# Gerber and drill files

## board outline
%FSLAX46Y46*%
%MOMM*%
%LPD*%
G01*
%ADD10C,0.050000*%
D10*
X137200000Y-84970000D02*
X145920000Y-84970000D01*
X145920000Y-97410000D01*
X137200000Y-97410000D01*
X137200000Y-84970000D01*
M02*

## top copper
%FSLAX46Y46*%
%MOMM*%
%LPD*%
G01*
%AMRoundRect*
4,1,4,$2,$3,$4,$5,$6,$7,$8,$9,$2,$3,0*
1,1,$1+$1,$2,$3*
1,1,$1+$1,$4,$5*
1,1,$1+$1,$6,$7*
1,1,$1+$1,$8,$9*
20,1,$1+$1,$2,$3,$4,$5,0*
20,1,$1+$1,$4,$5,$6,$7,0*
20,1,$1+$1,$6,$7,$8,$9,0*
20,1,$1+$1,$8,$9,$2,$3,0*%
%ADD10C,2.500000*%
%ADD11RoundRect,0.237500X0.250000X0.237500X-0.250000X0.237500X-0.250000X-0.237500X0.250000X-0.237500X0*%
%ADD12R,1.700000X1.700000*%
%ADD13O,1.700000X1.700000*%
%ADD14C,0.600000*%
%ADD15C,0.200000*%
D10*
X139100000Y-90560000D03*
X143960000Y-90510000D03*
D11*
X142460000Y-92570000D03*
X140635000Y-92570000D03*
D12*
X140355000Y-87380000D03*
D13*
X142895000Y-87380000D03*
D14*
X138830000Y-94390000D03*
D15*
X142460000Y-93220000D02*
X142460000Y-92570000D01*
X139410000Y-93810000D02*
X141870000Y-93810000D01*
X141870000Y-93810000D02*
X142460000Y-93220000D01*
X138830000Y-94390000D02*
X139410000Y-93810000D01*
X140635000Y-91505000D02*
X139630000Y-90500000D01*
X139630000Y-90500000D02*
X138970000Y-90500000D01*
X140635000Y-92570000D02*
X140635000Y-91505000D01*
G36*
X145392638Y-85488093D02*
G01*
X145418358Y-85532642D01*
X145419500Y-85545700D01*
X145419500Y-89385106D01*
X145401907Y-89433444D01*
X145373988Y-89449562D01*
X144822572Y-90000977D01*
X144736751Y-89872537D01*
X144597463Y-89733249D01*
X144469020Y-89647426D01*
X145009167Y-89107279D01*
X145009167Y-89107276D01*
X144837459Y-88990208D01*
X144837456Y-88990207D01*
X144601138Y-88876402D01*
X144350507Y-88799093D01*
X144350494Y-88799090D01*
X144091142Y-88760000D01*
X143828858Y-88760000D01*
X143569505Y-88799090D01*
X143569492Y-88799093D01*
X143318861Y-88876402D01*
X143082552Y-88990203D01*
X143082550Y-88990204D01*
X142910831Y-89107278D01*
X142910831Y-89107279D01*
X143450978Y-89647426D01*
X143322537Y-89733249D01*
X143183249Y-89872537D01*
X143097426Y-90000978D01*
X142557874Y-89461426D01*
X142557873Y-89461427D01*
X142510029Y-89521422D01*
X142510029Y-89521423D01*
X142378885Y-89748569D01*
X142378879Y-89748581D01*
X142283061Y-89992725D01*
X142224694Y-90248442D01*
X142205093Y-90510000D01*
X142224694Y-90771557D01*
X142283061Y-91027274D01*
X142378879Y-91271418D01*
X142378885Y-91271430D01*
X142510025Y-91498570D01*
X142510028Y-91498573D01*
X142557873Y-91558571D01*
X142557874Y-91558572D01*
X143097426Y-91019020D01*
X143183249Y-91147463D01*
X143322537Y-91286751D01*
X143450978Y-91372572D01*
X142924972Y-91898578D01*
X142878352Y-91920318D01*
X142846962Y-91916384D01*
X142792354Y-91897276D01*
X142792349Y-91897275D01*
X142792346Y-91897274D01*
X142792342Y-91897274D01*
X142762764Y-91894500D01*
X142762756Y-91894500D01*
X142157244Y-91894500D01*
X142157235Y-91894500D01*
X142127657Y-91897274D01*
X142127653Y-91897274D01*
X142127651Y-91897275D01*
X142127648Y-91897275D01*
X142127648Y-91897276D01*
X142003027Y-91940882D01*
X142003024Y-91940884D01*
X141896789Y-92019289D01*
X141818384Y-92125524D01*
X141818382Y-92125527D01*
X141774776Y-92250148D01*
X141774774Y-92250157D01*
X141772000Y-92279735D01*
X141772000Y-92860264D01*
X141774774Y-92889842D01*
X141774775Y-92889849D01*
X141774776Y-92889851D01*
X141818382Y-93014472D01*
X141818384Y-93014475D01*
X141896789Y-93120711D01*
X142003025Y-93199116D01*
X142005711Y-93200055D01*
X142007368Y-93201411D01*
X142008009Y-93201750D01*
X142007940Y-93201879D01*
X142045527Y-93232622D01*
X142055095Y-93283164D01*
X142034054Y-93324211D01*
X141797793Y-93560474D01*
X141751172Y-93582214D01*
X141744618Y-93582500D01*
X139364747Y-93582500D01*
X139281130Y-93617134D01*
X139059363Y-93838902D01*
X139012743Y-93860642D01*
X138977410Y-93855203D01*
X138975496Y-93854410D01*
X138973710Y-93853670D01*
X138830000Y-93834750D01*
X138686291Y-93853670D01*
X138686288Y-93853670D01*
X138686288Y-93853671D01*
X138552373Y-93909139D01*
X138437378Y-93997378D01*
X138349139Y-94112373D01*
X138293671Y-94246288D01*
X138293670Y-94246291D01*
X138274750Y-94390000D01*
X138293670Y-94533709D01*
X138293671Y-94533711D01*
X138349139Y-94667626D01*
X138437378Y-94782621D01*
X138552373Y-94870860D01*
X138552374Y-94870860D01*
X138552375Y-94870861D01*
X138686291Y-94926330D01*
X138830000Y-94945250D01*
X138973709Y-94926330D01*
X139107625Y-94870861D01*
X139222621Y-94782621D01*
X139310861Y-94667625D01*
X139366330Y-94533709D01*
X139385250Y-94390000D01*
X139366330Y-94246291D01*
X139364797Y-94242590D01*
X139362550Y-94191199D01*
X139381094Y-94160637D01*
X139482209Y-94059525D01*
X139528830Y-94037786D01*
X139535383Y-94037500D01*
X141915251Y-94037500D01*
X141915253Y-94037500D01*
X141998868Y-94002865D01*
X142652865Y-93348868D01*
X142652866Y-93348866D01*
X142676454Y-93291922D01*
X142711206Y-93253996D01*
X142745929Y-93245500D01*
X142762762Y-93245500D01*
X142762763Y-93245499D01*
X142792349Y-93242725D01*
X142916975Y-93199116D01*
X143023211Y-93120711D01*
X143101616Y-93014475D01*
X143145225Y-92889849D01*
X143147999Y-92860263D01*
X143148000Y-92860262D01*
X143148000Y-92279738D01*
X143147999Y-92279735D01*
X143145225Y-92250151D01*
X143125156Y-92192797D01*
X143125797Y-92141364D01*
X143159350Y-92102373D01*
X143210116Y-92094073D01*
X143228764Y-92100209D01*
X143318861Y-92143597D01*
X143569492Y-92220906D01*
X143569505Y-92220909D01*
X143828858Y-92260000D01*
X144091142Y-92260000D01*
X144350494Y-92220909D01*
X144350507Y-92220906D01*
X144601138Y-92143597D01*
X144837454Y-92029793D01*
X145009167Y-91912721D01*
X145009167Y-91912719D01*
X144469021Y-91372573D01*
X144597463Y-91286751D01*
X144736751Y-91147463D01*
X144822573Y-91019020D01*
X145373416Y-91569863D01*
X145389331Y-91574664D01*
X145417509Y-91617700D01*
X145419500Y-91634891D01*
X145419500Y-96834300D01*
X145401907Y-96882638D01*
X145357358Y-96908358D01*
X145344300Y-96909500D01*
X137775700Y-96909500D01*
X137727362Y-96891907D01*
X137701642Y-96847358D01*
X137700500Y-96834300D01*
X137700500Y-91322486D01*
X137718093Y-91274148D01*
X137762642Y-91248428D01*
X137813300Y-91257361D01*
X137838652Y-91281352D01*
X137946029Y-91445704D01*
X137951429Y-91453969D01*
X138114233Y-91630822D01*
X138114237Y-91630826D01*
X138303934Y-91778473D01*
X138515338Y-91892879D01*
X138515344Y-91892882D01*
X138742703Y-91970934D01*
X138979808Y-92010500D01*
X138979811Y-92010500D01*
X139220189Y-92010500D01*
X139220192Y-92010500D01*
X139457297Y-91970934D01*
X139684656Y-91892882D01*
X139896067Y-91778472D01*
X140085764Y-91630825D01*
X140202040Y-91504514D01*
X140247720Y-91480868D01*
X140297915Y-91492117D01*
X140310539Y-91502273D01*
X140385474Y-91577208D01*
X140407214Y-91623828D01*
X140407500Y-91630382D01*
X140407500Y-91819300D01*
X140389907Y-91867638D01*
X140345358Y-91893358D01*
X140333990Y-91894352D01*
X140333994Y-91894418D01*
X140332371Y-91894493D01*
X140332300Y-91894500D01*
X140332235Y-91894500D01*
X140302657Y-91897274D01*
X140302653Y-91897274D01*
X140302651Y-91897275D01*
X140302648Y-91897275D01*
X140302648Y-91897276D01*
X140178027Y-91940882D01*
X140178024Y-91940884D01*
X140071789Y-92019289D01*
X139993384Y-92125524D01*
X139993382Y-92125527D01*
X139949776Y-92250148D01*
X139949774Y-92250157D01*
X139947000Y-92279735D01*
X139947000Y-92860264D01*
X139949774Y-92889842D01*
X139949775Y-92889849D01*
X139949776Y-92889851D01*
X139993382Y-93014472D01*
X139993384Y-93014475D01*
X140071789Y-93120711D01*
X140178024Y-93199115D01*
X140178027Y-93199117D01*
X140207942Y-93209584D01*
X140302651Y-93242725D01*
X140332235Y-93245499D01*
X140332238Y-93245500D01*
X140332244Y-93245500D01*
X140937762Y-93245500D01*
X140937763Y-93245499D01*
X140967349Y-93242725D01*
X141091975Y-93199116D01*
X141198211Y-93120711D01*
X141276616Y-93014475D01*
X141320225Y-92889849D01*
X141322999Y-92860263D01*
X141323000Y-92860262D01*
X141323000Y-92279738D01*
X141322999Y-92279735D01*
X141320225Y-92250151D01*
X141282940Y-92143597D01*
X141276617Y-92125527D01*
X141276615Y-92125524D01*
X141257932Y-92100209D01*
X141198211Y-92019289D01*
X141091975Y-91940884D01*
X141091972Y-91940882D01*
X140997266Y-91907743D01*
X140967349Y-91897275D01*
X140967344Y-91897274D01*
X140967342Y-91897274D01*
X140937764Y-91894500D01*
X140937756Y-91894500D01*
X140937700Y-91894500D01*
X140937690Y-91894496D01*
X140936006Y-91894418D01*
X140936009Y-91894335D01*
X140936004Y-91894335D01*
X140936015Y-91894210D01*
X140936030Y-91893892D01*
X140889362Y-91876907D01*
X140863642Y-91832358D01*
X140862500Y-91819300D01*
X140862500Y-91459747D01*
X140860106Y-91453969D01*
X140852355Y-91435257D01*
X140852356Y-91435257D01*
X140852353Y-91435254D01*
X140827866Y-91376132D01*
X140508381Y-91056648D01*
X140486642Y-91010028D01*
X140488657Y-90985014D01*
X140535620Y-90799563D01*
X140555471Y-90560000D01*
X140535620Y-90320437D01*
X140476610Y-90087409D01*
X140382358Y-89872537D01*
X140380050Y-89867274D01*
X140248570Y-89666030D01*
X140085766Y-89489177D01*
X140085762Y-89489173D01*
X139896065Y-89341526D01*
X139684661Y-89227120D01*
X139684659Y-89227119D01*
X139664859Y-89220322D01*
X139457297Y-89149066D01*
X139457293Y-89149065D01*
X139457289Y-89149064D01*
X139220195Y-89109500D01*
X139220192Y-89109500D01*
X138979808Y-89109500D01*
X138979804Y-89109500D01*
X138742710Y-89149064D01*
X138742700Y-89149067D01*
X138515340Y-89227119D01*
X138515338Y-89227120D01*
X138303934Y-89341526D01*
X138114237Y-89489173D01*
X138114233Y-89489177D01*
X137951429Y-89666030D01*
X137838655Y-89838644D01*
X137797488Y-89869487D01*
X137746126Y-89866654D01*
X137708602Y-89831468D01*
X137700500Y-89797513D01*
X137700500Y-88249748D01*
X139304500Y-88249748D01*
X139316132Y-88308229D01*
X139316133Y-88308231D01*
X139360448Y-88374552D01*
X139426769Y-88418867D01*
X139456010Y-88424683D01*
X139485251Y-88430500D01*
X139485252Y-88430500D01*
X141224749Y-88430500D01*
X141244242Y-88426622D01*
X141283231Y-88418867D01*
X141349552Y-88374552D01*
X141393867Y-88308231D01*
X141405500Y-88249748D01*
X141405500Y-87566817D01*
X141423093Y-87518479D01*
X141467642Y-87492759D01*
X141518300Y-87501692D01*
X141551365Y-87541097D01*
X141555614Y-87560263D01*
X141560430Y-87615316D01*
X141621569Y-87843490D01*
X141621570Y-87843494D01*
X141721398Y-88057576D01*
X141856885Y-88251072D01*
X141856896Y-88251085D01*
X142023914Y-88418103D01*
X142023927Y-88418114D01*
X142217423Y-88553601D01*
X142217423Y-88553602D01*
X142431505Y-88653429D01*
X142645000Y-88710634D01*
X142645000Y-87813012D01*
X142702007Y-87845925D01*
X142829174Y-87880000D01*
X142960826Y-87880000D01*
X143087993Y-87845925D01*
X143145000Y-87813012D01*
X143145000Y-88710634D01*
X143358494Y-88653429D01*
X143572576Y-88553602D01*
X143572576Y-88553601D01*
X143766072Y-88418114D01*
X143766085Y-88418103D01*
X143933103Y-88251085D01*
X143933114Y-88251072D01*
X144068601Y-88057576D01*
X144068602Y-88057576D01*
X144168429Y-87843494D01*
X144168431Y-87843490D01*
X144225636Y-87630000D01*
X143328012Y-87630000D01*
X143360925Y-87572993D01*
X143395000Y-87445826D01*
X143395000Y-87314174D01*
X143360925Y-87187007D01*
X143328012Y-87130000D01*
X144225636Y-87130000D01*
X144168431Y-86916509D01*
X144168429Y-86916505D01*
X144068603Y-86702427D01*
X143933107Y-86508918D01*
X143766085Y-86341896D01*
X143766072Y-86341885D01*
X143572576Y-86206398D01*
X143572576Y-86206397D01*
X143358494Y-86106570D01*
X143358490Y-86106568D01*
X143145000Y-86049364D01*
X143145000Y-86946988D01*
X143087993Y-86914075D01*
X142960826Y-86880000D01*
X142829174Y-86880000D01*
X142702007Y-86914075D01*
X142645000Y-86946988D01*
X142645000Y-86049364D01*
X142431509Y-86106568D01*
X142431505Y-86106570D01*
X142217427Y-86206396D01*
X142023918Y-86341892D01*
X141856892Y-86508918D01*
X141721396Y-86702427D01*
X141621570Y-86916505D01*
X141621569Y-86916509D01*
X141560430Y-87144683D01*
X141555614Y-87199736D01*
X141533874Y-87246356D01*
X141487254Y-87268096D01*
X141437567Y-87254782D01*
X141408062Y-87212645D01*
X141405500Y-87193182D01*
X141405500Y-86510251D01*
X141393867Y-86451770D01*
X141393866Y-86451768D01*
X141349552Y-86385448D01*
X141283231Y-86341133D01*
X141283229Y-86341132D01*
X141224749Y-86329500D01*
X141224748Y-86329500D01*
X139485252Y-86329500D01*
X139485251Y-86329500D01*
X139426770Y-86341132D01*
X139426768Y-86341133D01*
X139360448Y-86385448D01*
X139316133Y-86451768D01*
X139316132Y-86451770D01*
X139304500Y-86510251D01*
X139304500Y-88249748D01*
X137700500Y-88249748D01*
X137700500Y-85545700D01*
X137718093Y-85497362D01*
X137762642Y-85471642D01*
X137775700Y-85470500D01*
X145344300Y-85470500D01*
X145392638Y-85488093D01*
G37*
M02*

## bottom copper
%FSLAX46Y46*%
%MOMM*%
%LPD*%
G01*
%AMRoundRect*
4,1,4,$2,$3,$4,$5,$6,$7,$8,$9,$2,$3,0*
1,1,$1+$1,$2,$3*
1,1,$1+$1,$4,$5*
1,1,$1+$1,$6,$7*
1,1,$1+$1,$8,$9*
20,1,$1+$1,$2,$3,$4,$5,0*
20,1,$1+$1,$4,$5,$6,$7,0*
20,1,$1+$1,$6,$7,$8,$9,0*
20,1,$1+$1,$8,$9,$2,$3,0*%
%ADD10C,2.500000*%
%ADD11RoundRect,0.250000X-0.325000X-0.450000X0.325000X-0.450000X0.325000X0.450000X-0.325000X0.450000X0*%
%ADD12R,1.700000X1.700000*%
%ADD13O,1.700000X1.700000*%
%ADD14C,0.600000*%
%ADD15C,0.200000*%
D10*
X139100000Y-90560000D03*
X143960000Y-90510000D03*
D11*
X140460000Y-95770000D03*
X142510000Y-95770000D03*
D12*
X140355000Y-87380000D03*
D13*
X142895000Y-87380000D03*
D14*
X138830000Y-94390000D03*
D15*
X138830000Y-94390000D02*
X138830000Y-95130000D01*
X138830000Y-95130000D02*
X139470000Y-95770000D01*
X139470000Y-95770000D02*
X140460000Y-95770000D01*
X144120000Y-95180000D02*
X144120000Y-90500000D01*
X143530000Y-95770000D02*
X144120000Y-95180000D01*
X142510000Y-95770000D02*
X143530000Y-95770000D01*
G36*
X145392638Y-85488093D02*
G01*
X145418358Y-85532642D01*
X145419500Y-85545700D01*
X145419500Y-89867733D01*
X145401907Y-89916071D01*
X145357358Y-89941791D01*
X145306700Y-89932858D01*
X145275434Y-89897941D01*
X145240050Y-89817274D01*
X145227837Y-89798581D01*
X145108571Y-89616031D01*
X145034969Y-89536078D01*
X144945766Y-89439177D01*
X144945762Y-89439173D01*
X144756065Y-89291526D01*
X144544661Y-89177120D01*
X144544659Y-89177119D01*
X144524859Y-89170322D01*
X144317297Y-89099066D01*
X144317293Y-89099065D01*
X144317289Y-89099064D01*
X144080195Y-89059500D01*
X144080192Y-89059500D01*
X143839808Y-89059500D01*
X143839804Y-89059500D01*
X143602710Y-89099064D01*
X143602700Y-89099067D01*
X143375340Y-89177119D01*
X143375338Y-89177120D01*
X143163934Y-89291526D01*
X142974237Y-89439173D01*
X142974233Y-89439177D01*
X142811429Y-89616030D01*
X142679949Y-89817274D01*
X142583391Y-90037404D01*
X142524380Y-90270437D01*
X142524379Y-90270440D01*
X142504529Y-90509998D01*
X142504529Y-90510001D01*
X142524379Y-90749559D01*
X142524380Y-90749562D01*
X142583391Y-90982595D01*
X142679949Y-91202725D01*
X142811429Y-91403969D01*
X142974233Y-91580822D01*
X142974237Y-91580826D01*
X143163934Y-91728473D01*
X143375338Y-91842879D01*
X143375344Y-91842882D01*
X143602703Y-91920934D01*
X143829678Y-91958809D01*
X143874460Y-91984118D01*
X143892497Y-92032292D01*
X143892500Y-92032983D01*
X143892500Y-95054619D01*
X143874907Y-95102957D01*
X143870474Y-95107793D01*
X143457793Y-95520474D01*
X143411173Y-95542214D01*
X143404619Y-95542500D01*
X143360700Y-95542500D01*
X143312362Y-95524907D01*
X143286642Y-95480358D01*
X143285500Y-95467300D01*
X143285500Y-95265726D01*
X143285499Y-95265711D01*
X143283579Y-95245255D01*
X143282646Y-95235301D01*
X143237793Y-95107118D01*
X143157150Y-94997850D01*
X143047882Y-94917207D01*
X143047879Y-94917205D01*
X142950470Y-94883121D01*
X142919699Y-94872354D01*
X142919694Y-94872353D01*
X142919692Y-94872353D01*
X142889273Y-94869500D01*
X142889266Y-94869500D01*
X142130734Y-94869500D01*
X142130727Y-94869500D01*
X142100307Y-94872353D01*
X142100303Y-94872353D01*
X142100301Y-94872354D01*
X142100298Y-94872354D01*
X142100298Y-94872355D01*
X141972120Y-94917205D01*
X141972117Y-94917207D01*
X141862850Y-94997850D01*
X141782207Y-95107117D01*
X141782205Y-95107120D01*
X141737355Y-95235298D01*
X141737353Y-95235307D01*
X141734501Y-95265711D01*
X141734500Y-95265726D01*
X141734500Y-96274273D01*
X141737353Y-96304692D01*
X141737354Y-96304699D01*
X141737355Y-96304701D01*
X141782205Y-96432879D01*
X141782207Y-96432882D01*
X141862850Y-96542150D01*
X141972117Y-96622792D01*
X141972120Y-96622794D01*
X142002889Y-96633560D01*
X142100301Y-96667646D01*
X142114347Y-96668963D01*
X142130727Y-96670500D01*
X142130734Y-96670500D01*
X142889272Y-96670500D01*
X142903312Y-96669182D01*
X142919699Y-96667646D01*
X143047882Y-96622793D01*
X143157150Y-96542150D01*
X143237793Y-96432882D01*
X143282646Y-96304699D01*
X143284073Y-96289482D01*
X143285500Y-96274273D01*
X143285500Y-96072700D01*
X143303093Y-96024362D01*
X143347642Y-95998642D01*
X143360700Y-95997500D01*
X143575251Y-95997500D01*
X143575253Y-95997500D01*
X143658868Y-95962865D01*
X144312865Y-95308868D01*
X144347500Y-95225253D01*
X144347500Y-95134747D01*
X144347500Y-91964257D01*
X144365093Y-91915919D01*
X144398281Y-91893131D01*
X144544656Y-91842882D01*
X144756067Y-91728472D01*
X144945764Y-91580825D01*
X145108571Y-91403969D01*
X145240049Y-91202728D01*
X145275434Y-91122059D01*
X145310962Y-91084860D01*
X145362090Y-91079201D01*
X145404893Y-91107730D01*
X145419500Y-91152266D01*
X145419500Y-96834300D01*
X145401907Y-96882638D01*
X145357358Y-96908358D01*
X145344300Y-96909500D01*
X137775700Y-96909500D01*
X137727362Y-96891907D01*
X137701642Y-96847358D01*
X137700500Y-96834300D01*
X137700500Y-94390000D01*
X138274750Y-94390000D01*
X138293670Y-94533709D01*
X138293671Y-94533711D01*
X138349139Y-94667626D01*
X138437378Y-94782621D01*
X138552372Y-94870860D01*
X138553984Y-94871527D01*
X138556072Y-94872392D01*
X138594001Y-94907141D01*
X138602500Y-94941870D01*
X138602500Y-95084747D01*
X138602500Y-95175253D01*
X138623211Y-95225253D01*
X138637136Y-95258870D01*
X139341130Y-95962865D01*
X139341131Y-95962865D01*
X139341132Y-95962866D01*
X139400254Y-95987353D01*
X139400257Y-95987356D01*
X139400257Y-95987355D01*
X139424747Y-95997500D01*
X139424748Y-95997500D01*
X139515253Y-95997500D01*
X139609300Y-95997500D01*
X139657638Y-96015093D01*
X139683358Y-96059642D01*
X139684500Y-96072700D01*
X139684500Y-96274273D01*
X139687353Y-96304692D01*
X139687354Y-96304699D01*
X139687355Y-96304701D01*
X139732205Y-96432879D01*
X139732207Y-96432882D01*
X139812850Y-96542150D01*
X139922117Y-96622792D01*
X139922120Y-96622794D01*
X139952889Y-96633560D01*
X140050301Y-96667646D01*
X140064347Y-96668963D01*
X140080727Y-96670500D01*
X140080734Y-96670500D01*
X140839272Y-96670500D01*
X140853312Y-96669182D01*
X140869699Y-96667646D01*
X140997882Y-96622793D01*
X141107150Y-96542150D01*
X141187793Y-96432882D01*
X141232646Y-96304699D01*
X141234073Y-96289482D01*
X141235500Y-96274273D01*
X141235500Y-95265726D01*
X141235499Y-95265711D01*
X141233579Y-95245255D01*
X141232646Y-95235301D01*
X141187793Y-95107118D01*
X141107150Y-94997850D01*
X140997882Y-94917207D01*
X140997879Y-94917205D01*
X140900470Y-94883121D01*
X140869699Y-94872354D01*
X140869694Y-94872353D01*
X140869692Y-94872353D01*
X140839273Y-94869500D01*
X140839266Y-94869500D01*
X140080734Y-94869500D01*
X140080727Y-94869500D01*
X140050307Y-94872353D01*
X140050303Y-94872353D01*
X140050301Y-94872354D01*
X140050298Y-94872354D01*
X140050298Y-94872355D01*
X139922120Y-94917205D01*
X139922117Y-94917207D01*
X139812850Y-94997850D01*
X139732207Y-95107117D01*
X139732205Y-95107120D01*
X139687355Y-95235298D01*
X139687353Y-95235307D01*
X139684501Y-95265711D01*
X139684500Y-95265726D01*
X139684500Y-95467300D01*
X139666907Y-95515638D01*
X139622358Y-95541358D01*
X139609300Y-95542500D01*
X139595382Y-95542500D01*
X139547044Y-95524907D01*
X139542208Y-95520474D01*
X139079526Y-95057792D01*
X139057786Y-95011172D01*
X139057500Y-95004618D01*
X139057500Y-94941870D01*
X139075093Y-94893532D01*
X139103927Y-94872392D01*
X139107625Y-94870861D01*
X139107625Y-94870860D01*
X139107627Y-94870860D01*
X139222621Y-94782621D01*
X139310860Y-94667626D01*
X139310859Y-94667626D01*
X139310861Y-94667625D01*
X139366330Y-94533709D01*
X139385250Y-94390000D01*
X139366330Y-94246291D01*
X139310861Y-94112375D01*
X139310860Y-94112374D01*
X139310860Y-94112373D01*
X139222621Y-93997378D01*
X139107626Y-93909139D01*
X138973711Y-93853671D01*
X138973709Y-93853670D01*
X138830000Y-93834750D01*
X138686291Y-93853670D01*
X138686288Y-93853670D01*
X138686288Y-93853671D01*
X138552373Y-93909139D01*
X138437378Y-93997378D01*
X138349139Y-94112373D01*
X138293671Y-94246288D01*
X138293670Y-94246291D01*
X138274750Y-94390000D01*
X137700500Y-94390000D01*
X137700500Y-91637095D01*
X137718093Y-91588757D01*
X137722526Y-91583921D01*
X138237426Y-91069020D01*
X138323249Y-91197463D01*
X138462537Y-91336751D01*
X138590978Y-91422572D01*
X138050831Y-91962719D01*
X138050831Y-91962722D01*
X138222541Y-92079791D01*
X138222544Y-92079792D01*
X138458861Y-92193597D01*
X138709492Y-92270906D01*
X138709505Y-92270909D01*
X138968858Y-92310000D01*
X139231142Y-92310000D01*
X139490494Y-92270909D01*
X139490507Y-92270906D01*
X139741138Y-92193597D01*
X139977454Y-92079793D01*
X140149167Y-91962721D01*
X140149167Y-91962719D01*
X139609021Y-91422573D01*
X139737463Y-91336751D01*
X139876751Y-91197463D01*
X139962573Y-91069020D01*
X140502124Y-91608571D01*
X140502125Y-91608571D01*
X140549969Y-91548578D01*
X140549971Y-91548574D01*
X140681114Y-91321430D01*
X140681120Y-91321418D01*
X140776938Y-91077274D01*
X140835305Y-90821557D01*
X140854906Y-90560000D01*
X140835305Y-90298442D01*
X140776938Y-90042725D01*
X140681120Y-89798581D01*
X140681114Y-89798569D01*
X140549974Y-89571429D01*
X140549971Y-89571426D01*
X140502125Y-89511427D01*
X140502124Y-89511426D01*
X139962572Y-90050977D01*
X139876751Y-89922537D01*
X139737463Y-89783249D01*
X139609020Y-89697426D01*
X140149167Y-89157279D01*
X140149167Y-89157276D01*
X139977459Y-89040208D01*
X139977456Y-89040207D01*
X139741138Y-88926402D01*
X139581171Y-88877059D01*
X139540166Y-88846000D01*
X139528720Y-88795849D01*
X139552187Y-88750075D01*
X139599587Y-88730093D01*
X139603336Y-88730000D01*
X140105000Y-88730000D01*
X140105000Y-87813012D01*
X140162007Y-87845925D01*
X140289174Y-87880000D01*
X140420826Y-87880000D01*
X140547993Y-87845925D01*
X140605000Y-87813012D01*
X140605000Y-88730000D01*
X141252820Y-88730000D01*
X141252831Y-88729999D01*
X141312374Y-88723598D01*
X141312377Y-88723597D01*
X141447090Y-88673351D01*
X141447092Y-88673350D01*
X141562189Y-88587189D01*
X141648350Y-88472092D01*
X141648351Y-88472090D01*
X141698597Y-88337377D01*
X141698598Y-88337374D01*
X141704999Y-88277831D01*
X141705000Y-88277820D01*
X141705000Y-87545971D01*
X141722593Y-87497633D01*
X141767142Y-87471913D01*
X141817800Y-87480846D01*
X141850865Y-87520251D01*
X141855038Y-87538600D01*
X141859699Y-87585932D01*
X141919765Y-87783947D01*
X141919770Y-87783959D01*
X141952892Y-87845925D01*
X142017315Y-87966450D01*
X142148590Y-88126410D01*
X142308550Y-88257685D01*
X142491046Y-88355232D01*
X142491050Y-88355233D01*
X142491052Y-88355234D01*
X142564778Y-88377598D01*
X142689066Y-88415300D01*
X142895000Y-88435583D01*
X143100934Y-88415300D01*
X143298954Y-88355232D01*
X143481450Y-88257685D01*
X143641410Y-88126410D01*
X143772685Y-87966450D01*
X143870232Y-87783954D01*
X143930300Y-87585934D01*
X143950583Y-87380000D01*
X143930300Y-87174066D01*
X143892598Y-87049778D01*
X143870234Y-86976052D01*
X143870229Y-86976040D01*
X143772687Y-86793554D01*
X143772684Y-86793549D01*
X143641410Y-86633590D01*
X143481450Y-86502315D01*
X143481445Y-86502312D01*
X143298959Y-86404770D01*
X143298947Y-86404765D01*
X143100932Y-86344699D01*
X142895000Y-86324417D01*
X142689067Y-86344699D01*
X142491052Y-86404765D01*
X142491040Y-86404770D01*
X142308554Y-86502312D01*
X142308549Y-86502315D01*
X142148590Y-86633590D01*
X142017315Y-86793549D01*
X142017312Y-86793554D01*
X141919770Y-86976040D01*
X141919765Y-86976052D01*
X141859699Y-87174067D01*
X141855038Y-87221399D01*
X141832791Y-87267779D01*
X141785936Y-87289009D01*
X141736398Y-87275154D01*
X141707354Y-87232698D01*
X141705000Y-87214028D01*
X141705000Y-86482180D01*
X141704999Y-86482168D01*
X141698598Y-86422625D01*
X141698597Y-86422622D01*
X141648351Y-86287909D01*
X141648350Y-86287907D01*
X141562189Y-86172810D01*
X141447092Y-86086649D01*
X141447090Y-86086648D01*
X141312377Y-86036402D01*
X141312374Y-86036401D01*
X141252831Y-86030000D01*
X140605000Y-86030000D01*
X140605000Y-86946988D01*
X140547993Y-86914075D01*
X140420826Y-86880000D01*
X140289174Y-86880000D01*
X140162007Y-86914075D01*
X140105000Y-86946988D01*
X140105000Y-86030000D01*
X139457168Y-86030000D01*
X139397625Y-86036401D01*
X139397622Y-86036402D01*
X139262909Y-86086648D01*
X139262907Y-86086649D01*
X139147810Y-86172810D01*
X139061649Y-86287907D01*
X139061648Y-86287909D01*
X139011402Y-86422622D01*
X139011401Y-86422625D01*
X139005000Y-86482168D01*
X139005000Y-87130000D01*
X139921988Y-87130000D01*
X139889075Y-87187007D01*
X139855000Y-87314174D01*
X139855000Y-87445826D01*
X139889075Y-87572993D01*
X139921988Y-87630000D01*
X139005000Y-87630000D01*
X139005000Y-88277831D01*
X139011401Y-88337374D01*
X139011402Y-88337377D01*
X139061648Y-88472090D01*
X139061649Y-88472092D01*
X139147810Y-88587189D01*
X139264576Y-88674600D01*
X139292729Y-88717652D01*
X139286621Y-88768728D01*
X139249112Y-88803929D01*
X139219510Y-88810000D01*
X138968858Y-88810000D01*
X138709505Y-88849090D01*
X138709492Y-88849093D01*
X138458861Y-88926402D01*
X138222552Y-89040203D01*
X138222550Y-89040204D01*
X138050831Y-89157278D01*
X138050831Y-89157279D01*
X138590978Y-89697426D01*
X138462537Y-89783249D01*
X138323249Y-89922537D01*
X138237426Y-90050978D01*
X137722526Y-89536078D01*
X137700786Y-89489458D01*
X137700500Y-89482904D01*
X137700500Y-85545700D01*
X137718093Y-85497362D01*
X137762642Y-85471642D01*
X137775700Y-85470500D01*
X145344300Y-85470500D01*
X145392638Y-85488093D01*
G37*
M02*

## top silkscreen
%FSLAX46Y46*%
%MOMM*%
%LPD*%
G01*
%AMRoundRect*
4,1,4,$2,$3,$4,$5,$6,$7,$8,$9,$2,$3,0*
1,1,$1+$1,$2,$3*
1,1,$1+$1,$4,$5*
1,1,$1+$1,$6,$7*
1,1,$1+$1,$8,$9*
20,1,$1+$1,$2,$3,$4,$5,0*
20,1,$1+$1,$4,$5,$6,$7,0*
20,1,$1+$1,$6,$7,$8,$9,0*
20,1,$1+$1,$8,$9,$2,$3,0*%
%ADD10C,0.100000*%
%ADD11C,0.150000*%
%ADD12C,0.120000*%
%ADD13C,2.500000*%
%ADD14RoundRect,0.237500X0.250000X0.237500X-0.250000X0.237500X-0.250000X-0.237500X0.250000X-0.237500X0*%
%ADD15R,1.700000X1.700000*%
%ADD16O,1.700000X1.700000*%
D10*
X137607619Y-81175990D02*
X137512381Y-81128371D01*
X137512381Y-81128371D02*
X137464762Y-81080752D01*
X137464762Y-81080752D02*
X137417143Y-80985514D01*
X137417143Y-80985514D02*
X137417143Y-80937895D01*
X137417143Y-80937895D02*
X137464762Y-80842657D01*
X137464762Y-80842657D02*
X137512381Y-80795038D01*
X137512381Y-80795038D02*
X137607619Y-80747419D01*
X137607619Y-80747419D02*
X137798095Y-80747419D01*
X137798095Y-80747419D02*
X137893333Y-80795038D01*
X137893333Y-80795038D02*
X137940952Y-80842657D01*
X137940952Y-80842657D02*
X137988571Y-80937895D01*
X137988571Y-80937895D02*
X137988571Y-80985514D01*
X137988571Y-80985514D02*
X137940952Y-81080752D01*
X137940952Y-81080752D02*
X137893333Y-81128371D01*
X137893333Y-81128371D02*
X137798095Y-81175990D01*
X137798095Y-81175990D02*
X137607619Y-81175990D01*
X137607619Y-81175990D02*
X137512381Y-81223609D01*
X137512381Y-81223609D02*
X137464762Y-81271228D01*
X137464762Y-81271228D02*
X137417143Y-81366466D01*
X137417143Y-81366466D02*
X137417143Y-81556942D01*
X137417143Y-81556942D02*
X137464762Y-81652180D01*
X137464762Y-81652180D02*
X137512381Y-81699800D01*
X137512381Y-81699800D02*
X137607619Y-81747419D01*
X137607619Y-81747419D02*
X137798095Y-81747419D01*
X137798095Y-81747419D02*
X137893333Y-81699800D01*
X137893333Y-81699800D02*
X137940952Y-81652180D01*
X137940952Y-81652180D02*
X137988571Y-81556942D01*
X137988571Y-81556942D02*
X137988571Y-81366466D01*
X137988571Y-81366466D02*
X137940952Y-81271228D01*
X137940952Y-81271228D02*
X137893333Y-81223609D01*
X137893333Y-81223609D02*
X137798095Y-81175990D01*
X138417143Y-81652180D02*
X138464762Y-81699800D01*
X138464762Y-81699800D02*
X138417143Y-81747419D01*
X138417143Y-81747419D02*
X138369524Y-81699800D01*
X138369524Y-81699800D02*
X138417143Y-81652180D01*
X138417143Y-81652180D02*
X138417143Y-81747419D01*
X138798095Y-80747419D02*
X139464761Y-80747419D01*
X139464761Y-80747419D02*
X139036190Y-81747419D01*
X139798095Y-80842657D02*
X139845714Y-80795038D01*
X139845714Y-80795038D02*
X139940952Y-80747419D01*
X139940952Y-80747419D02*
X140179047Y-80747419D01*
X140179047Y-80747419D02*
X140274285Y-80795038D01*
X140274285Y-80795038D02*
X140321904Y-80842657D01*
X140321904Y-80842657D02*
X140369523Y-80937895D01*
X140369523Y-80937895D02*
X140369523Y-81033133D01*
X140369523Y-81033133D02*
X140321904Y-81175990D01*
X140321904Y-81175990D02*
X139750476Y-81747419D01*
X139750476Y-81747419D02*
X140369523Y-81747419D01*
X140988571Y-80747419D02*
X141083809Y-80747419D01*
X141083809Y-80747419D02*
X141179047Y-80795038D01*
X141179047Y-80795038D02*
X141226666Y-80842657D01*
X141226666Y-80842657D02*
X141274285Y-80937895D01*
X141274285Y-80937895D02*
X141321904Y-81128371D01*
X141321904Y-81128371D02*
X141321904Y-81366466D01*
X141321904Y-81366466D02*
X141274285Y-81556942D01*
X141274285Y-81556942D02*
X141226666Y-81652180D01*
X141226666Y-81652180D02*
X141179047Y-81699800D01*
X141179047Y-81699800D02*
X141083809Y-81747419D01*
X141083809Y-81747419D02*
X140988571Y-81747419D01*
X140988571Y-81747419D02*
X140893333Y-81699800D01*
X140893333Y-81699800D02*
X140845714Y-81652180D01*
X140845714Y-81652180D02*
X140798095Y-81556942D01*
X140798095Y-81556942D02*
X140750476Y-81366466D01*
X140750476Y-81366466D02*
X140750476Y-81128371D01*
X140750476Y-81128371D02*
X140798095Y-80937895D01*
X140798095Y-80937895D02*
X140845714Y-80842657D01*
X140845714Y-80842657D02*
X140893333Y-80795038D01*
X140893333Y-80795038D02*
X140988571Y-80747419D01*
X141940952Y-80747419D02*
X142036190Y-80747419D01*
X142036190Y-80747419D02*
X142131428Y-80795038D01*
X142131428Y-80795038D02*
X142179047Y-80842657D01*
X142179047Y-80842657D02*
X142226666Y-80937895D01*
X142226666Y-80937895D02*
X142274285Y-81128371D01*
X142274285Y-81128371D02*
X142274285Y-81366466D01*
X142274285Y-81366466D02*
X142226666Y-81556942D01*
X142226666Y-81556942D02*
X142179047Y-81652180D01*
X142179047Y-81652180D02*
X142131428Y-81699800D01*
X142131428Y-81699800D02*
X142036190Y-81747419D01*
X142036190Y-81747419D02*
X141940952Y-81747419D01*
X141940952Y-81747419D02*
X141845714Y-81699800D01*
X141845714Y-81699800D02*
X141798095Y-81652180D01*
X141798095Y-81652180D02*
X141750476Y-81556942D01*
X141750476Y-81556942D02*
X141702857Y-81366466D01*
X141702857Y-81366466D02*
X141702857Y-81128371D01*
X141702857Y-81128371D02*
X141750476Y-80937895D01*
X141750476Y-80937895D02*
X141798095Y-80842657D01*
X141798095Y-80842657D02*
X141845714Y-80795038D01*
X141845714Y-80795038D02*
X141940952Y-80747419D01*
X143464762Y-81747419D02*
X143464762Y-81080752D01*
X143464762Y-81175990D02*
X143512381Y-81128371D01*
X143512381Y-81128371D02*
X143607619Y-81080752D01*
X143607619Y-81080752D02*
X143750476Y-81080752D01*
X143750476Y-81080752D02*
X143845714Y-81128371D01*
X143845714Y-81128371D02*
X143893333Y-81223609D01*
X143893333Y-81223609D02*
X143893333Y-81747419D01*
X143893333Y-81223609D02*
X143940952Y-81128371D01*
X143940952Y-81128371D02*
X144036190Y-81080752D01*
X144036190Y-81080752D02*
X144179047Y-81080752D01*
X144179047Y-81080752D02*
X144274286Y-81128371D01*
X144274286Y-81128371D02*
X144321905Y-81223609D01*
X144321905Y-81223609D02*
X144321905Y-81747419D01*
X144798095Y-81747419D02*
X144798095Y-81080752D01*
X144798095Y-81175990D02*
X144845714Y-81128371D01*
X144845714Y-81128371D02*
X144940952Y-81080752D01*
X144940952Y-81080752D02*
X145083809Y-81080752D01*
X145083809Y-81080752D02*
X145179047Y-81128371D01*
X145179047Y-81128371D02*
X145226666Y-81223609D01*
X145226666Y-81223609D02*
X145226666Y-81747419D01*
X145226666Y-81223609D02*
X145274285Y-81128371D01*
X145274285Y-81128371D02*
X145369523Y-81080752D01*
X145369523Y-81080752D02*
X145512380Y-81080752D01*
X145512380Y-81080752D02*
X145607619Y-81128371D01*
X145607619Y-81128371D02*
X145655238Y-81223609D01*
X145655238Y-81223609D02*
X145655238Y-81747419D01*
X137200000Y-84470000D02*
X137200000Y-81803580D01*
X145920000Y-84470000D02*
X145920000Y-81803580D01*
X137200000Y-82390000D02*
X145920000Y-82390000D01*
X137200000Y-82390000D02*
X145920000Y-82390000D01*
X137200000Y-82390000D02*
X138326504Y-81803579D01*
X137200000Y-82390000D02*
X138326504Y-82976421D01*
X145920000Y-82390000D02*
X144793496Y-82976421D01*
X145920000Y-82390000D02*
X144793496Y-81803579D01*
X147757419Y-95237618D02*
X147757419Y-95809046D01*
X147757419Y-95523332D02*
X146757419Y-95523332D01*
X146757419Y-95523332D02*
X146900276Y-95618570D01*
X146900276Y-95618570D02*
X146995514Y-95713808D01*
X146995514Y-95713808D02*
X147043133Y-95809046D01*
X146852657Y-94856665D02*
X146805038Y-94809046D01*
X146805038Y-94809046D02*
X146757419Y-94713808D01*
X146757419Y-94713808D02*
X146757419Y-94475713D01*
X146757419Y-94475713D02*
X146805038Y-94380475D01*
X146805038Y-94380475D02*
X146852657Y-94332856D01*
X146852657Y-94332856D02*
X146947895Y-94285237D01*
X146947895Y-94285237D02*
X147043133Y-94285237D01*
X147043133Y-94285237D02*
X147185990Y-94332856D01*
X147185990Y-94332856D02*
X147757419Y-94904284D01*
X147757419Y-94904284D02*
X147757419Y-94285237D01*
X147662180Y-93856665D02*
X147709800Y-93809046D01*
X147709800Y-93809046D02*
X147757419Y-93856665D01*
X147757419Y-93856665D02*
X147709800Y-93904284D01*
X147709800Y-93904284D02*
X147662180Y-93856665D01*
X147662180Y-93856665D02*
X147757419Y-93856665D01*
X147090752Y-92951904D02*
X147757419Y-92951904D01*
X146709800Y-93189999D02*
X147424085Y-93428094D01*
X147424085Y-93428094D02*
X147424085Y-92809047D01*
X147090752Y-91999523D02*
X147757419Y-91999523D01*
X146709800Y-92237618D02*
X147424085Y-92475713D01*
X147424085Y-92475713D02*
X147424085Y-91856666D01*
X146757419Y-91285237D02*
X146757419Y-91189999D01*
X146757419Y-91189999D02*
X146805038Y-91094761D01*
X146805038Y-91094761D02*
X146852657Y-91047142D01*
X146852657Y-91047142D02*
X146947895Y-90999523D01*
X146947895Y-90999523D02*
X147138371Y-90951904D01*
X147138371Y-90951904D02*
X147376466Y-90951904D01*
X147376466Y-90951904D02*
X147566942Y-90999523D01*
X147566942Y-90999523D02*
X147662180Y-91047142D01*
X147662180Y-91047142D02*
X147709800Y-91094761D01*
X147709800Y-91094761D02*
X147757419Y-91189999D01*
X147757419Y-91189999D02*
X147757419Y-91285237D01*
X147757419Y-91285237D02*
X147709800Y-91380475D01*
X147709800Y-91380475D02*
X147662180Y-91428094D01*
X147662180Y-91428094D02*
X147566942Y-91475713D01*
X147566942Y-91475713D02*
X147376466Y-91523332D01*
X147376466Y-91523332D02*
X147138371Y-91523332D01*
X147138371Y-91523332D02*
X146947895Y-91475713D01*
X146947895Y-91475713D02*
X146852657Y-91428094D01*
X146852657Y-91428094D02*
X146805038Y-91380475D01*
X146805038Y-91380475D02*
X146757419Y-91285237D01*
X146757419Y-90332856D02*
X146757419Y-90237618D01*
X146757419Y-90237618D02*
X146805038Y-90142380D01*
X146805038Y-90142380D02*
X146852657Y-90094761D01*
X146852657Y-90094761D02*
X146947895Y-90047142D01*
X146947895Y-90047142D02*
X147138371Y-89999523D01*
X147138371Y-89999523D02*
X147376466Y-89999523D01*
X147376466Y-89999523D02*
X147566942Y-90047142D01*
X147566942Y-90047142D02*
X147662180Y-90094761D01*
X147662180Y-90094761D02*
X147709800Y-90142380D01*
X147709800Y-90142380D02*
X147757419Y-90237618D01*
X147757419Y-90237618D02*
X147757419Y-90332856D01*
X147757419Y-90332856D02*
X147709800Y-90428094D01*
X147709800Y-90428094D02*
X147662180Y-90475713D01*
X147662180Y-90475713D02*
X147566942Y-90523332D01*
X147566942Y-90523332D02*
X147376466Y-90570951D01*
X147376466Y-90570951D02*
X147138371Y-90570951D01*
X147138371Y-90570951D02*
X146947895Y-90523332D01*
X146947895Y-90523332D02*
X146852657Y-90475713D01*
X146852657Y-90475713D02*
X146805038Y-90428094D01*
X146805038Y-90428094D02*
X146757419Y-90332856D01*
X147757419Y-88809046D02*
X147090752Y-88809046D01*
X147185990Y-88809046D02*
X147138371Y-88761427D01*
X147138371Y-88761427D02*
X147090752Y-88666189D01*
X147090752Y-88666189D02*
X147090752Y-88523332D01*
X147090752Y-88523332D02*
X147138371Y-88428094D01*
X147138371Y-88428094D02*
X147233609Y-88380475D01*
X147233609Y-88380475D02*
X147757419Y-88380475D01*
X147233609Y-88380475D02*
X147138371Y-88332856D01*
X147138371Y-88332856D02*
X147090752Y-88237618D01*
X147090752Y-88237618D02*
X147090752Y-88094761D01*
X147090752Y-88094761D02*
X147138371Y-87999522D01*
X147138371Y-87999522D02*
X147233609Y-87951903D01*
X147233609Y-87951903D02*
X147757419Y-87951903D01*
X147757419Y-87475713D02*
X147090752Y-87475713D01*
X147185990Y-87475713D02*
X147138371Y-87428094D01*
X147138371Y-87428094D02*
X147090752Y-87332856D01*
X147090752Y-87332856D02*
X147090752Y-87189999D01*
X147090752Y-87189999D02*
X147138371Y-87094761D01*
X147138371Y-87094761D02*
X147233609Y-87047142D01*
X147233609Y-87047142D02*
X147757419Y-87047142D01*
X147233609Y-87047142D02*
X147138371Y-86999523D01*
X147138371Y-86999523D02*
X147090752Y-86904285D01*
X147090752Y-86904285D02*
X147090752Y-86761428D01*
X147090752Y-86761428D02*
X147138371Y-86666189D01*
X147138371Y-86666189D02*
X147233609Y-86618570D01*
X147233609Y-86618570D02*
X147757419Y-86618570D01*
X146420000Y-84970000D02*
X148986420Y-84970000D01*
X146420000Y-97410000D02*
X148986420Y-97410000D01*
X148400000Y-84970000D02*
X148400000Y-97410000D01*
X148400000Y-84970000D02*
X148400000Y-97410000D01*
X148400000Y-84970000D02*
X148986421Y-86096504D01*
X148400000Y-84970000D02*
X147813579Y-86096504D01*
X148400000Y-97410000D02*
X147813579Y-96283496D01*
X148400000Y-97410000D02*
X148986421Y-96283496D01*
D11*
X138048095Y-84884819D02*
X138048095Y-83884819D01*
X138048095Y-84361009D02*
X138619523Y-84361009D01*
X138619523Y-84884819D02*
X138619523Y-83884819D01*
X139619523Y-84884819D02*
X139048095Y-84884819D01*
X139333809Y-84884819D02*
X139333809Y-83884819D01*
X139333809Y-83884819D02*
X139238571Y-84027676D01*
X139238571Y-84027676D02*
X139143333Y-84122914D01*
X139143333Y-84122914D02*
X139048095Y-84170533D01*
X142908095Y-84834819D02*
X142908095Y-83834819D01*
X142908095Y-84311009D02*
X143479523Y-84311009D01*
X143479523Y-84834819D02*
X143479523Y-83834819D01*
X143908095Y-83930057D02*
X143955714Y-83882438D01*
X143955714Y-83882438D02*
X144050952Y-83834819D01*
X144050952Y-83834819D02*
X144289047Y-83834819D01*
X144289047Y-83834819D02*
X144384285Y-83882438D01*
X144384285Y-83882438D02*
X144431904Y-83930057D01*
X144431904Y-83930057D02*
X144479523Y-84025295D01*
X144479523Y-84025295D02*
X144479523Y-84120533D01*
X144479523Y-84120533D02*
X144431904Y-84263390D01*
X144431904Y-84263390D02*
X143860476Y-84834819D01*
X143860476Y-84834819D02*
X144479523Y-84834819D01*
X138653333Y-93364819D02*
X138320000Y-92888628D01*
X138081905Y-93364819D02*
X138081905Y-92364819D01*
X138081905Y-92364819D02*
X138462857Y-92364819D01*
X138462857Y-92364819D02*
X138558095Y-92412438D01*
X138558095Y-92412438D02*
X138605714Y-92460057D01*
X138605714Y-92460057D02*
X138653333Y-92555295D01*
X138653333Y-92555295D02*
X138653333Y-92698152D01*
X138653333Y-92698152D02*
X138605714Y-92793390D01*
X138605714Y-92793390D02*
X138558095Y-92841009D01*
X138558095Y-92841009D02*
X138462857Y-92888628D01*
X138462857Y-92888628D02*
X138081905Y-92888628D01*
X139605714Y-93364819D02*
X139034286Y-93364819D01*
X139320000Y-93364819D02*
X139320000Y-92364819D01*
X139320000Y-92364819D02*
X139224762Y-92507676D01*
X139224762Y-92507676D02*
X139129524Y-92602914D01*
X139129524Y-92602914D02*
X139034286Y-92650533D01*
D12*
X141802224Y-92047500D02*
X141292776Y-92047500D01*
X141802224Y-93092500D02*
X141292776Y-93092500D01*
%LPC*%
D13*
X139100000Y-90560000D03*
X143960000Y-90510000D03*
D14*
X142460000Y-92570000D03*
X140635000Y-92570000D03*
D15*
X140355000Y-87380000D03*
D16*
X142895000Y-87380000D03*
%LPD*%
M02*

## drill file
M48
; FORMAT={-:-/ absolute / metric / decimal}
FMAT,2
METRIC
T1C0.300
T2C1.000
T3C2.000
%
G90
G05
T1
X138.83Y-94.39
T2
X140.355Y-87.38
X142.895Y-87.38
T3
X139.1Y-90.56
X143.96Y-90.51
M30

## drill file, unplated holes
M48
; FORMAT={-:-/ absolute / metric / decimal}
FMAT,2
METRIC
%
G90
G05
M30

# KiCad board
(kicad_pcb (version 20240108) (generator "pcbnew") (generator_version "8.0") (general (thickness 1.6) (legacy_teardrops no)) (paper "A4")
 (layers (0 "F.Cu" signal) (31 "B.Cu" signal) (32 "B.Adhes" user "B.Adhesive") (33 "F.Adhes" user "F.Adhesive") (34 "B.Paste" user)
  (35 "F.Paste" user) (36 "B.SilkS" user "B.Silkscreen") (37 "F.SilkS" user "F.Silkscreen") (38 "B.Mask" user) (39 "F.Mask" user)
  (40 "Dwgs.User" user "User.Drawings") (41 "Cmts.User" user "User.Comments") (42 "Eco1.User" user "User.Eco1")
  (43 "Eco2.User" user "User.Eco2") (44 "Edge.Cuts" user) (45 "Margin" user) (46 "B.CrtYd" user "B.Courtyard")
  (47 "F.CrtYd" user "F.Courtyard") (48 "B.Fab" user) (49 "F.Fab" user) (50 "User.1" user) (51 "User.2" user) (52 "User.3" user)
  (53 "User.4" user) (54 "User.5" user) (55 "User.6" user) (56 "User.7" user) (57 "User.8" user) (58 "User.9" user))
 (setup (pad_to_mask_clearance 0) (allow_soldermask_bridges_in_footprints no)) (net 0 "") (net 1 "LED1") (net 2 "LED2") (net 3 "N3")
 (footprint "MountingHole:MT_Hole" (layer "F.Cu") (at 139.1 90.56)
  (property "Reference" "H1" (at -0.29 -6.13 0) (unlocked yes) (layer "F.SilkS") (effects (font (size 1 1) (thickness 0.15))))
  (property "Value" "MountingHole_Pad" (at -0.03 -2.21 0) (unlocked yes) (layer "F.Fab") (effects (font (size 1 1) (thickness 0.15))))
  (pad "1" thru_hole circle (at 0 0) (size 2.5 2.5) (drill 2) (layers "*.Cu" "*.Mask") (remove_unused_layers no) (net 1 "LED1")))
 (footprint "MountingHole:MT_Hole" (layer "F.Cu") (at 143.96 90.51)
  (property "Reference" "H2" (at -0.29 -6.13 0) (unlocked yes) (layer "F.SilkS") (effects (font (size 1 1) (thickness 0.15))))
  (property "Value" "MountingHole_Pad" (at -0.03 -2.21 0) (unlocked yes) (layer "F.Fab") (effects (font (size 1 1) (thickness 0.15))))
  (pad "1" thru_hole circle (at 0 0) (size 2.5 2.5) (drill 2) (layers "*.Cu" "*.Mask") (remove_unused_layers no) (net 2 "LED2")))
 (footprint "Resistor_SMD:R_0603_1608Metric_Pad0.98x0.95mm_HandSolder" (layer "F.Cu") (at 141.5475 92.57 180)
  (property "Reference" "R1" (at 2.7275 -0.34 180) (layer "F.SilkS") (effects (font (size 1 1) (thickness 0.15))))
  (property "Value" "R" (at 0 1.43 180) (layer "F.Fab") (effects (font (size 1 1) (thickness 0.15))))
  (fp_line (start -0.254724 0.5225) (end 0.254724 0.5225) (stroke (width 0.12) (type solid)) (layer "F.SilkS"))
  (fp_line (start -0.254724 -0.5225) (end 0.254724 -0.5225) (stroke (width 0.12) (type solid)) (layer "F.SilkS"))
  (pad "1" smd roundrect (at -0.9125 0 180) (size 0.975 0.95) (layers "F.Cu" "F.Paste" "F.Mask") (roundrect_rratio 0.25) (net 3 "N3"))
  (pad "2" smd roundrect (at 0.9125 0 180) (size 0.975 0.95) (layers "F.Cu" "F.Paste" "F.Mask") (roundrect_rratio 0.25) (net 1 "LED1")))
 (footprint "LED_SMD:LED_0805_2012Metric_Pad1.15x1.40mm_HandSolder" (layer "B.Cu") (at 141.485 95.77)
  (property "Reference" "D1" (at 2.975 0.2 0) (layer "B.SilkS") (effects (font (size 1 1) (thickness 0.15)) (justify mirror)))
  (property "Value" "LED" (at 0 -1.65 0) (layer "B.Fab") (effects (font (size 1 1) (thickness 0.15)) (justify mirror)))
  (pad "1" smd roundrect (at -1.025 0) (size 1.15 1.4) (layers "B.Cu" "B.Paste" "B.Mask") (roundrect_rratio 0.217391) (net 3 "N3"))
  (pad "2" smd roundrect (at 1.025 0) (size 1.15 1.4) (layers "B.Cu" "B.Paste" "B.Mask") (roundrect_rratio 0.217391) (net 2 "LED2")))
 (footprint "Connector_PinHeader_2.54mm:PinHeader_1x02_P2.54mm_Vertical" (layer "B.Cu") (at 140.355 87.38 -90)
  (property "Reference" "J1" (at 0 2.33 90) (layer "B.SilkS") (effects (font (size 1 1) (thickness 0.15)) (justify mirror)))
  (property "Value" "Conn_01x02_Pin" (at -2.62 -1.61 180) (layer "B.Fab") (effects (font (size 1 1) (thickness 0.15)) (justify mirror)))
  (pad "1" thru_hole rect (at 0 0 270) (size 1.7 1.7) (drill 1) (layers "*.Cu" "*.Mask") (remove_unused_layers no) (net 1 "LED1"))
  (pad "2" thru_hole oval (at 0 -2.54 270) (size 1.7 1.7) (drill 1) (layers "*.Cu" "*.Mask") (remove_unused_layers no) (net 2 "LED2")))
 (gr_rect (start 137.2 84.97) (end 145.92 97.41) (stroke (width 0.05) (type default)) (fill none) (layer "Edge.Cuts"))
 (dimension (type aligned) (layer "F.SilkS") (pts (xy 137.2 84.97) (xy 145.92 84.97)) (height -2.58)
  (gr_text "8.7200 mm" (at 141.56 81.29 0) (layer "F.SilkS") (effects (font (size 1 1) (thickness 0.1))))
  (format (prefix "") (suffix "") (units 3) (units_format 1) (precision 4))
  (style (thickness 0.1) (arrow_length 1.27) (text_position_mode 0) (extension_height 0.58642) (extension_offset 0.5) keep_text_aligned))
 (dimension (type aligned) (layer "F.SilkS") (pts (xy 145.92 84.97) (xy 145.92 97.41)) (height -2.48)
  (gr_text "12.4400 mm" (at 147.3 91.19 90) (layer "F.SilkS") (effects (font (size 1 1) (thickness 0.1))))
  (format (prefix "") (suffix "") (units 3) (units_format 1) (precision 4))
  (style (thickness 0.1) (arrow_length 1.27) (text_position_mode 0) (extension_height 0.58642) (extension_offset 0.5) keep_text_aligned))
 (segment (start 142.46 93.22) (end 142.46 92.57) (width 0.2) (layer "F.Cu") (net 3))
 (segment (start 139.41 93.81) (end 141.87 93.81) (width 0.2) (layer "F.Cu") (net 3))
 (segment (start 141.87 93.81) (end 142.46 93.22) (width 0.2) (layer "F.Cu") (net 3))
 (segment (start 138.83 94.39) (end 139.41 93.81) (width 0.2) (layer "F.Cu") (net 3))
 (via (at 138.83 94.39) (size 0.6) (drill 0.3) (layers "F.Cu" "B.Cu") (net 3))
 (segment (start 138.83 94.39) (end 138.83 95.13) (width 0.2) (layer "B.Cu") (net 3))
 (segment (start 138.83 95.13) (end 139.47 95.77) (width 0.2) (layer "B.Cu") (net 3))
 (segment (start 139.47 95.77) (end 140.46 95.77) (width 0.2) (layer "B.Cu") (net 3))
 (segment (start 144.12 95.18) (end 144.12 90.5) (width 0.2) (layer "B.Cu") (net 2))
 (segment (start 143.53 95.77) (end 144.12 95.18) (width 0.2) (layer "B.Cu") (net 2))
 (segment (start 142.51 95.77) (end 143.53 95.77) (width 0.2) (layer "B.Cu") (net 2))
 (segment (start 140.635 91.505) (end 139.63 90.5) (width 0.2) (layer "F.Cu") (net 1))
 (segment (start 139.63 90.5) (end 138.97 90.5) (width 0.2) (layer "F.Cu") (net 1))
 (segment (start 140.635 92.57) (end 140.635 91.505) (width 0.2) (layer "F.Cu") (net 1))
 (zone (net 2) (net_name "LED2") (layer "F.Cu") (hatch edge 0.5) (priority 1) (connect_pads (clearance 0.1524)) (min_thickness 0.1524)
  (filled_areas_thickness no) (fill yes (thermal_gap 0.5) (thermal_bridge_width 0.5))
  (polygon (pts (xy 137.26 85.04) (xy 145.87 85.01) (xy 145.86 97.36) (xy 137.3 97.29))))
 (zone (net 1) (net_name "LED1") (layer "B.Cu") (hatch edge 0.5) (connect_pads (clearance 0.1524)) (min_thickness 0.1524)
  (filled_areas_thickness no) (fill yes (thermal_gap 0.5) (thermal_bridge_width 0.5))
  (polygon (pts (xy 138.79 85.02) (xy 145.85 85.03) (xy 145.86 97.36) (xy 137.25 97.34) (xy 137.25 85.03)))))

